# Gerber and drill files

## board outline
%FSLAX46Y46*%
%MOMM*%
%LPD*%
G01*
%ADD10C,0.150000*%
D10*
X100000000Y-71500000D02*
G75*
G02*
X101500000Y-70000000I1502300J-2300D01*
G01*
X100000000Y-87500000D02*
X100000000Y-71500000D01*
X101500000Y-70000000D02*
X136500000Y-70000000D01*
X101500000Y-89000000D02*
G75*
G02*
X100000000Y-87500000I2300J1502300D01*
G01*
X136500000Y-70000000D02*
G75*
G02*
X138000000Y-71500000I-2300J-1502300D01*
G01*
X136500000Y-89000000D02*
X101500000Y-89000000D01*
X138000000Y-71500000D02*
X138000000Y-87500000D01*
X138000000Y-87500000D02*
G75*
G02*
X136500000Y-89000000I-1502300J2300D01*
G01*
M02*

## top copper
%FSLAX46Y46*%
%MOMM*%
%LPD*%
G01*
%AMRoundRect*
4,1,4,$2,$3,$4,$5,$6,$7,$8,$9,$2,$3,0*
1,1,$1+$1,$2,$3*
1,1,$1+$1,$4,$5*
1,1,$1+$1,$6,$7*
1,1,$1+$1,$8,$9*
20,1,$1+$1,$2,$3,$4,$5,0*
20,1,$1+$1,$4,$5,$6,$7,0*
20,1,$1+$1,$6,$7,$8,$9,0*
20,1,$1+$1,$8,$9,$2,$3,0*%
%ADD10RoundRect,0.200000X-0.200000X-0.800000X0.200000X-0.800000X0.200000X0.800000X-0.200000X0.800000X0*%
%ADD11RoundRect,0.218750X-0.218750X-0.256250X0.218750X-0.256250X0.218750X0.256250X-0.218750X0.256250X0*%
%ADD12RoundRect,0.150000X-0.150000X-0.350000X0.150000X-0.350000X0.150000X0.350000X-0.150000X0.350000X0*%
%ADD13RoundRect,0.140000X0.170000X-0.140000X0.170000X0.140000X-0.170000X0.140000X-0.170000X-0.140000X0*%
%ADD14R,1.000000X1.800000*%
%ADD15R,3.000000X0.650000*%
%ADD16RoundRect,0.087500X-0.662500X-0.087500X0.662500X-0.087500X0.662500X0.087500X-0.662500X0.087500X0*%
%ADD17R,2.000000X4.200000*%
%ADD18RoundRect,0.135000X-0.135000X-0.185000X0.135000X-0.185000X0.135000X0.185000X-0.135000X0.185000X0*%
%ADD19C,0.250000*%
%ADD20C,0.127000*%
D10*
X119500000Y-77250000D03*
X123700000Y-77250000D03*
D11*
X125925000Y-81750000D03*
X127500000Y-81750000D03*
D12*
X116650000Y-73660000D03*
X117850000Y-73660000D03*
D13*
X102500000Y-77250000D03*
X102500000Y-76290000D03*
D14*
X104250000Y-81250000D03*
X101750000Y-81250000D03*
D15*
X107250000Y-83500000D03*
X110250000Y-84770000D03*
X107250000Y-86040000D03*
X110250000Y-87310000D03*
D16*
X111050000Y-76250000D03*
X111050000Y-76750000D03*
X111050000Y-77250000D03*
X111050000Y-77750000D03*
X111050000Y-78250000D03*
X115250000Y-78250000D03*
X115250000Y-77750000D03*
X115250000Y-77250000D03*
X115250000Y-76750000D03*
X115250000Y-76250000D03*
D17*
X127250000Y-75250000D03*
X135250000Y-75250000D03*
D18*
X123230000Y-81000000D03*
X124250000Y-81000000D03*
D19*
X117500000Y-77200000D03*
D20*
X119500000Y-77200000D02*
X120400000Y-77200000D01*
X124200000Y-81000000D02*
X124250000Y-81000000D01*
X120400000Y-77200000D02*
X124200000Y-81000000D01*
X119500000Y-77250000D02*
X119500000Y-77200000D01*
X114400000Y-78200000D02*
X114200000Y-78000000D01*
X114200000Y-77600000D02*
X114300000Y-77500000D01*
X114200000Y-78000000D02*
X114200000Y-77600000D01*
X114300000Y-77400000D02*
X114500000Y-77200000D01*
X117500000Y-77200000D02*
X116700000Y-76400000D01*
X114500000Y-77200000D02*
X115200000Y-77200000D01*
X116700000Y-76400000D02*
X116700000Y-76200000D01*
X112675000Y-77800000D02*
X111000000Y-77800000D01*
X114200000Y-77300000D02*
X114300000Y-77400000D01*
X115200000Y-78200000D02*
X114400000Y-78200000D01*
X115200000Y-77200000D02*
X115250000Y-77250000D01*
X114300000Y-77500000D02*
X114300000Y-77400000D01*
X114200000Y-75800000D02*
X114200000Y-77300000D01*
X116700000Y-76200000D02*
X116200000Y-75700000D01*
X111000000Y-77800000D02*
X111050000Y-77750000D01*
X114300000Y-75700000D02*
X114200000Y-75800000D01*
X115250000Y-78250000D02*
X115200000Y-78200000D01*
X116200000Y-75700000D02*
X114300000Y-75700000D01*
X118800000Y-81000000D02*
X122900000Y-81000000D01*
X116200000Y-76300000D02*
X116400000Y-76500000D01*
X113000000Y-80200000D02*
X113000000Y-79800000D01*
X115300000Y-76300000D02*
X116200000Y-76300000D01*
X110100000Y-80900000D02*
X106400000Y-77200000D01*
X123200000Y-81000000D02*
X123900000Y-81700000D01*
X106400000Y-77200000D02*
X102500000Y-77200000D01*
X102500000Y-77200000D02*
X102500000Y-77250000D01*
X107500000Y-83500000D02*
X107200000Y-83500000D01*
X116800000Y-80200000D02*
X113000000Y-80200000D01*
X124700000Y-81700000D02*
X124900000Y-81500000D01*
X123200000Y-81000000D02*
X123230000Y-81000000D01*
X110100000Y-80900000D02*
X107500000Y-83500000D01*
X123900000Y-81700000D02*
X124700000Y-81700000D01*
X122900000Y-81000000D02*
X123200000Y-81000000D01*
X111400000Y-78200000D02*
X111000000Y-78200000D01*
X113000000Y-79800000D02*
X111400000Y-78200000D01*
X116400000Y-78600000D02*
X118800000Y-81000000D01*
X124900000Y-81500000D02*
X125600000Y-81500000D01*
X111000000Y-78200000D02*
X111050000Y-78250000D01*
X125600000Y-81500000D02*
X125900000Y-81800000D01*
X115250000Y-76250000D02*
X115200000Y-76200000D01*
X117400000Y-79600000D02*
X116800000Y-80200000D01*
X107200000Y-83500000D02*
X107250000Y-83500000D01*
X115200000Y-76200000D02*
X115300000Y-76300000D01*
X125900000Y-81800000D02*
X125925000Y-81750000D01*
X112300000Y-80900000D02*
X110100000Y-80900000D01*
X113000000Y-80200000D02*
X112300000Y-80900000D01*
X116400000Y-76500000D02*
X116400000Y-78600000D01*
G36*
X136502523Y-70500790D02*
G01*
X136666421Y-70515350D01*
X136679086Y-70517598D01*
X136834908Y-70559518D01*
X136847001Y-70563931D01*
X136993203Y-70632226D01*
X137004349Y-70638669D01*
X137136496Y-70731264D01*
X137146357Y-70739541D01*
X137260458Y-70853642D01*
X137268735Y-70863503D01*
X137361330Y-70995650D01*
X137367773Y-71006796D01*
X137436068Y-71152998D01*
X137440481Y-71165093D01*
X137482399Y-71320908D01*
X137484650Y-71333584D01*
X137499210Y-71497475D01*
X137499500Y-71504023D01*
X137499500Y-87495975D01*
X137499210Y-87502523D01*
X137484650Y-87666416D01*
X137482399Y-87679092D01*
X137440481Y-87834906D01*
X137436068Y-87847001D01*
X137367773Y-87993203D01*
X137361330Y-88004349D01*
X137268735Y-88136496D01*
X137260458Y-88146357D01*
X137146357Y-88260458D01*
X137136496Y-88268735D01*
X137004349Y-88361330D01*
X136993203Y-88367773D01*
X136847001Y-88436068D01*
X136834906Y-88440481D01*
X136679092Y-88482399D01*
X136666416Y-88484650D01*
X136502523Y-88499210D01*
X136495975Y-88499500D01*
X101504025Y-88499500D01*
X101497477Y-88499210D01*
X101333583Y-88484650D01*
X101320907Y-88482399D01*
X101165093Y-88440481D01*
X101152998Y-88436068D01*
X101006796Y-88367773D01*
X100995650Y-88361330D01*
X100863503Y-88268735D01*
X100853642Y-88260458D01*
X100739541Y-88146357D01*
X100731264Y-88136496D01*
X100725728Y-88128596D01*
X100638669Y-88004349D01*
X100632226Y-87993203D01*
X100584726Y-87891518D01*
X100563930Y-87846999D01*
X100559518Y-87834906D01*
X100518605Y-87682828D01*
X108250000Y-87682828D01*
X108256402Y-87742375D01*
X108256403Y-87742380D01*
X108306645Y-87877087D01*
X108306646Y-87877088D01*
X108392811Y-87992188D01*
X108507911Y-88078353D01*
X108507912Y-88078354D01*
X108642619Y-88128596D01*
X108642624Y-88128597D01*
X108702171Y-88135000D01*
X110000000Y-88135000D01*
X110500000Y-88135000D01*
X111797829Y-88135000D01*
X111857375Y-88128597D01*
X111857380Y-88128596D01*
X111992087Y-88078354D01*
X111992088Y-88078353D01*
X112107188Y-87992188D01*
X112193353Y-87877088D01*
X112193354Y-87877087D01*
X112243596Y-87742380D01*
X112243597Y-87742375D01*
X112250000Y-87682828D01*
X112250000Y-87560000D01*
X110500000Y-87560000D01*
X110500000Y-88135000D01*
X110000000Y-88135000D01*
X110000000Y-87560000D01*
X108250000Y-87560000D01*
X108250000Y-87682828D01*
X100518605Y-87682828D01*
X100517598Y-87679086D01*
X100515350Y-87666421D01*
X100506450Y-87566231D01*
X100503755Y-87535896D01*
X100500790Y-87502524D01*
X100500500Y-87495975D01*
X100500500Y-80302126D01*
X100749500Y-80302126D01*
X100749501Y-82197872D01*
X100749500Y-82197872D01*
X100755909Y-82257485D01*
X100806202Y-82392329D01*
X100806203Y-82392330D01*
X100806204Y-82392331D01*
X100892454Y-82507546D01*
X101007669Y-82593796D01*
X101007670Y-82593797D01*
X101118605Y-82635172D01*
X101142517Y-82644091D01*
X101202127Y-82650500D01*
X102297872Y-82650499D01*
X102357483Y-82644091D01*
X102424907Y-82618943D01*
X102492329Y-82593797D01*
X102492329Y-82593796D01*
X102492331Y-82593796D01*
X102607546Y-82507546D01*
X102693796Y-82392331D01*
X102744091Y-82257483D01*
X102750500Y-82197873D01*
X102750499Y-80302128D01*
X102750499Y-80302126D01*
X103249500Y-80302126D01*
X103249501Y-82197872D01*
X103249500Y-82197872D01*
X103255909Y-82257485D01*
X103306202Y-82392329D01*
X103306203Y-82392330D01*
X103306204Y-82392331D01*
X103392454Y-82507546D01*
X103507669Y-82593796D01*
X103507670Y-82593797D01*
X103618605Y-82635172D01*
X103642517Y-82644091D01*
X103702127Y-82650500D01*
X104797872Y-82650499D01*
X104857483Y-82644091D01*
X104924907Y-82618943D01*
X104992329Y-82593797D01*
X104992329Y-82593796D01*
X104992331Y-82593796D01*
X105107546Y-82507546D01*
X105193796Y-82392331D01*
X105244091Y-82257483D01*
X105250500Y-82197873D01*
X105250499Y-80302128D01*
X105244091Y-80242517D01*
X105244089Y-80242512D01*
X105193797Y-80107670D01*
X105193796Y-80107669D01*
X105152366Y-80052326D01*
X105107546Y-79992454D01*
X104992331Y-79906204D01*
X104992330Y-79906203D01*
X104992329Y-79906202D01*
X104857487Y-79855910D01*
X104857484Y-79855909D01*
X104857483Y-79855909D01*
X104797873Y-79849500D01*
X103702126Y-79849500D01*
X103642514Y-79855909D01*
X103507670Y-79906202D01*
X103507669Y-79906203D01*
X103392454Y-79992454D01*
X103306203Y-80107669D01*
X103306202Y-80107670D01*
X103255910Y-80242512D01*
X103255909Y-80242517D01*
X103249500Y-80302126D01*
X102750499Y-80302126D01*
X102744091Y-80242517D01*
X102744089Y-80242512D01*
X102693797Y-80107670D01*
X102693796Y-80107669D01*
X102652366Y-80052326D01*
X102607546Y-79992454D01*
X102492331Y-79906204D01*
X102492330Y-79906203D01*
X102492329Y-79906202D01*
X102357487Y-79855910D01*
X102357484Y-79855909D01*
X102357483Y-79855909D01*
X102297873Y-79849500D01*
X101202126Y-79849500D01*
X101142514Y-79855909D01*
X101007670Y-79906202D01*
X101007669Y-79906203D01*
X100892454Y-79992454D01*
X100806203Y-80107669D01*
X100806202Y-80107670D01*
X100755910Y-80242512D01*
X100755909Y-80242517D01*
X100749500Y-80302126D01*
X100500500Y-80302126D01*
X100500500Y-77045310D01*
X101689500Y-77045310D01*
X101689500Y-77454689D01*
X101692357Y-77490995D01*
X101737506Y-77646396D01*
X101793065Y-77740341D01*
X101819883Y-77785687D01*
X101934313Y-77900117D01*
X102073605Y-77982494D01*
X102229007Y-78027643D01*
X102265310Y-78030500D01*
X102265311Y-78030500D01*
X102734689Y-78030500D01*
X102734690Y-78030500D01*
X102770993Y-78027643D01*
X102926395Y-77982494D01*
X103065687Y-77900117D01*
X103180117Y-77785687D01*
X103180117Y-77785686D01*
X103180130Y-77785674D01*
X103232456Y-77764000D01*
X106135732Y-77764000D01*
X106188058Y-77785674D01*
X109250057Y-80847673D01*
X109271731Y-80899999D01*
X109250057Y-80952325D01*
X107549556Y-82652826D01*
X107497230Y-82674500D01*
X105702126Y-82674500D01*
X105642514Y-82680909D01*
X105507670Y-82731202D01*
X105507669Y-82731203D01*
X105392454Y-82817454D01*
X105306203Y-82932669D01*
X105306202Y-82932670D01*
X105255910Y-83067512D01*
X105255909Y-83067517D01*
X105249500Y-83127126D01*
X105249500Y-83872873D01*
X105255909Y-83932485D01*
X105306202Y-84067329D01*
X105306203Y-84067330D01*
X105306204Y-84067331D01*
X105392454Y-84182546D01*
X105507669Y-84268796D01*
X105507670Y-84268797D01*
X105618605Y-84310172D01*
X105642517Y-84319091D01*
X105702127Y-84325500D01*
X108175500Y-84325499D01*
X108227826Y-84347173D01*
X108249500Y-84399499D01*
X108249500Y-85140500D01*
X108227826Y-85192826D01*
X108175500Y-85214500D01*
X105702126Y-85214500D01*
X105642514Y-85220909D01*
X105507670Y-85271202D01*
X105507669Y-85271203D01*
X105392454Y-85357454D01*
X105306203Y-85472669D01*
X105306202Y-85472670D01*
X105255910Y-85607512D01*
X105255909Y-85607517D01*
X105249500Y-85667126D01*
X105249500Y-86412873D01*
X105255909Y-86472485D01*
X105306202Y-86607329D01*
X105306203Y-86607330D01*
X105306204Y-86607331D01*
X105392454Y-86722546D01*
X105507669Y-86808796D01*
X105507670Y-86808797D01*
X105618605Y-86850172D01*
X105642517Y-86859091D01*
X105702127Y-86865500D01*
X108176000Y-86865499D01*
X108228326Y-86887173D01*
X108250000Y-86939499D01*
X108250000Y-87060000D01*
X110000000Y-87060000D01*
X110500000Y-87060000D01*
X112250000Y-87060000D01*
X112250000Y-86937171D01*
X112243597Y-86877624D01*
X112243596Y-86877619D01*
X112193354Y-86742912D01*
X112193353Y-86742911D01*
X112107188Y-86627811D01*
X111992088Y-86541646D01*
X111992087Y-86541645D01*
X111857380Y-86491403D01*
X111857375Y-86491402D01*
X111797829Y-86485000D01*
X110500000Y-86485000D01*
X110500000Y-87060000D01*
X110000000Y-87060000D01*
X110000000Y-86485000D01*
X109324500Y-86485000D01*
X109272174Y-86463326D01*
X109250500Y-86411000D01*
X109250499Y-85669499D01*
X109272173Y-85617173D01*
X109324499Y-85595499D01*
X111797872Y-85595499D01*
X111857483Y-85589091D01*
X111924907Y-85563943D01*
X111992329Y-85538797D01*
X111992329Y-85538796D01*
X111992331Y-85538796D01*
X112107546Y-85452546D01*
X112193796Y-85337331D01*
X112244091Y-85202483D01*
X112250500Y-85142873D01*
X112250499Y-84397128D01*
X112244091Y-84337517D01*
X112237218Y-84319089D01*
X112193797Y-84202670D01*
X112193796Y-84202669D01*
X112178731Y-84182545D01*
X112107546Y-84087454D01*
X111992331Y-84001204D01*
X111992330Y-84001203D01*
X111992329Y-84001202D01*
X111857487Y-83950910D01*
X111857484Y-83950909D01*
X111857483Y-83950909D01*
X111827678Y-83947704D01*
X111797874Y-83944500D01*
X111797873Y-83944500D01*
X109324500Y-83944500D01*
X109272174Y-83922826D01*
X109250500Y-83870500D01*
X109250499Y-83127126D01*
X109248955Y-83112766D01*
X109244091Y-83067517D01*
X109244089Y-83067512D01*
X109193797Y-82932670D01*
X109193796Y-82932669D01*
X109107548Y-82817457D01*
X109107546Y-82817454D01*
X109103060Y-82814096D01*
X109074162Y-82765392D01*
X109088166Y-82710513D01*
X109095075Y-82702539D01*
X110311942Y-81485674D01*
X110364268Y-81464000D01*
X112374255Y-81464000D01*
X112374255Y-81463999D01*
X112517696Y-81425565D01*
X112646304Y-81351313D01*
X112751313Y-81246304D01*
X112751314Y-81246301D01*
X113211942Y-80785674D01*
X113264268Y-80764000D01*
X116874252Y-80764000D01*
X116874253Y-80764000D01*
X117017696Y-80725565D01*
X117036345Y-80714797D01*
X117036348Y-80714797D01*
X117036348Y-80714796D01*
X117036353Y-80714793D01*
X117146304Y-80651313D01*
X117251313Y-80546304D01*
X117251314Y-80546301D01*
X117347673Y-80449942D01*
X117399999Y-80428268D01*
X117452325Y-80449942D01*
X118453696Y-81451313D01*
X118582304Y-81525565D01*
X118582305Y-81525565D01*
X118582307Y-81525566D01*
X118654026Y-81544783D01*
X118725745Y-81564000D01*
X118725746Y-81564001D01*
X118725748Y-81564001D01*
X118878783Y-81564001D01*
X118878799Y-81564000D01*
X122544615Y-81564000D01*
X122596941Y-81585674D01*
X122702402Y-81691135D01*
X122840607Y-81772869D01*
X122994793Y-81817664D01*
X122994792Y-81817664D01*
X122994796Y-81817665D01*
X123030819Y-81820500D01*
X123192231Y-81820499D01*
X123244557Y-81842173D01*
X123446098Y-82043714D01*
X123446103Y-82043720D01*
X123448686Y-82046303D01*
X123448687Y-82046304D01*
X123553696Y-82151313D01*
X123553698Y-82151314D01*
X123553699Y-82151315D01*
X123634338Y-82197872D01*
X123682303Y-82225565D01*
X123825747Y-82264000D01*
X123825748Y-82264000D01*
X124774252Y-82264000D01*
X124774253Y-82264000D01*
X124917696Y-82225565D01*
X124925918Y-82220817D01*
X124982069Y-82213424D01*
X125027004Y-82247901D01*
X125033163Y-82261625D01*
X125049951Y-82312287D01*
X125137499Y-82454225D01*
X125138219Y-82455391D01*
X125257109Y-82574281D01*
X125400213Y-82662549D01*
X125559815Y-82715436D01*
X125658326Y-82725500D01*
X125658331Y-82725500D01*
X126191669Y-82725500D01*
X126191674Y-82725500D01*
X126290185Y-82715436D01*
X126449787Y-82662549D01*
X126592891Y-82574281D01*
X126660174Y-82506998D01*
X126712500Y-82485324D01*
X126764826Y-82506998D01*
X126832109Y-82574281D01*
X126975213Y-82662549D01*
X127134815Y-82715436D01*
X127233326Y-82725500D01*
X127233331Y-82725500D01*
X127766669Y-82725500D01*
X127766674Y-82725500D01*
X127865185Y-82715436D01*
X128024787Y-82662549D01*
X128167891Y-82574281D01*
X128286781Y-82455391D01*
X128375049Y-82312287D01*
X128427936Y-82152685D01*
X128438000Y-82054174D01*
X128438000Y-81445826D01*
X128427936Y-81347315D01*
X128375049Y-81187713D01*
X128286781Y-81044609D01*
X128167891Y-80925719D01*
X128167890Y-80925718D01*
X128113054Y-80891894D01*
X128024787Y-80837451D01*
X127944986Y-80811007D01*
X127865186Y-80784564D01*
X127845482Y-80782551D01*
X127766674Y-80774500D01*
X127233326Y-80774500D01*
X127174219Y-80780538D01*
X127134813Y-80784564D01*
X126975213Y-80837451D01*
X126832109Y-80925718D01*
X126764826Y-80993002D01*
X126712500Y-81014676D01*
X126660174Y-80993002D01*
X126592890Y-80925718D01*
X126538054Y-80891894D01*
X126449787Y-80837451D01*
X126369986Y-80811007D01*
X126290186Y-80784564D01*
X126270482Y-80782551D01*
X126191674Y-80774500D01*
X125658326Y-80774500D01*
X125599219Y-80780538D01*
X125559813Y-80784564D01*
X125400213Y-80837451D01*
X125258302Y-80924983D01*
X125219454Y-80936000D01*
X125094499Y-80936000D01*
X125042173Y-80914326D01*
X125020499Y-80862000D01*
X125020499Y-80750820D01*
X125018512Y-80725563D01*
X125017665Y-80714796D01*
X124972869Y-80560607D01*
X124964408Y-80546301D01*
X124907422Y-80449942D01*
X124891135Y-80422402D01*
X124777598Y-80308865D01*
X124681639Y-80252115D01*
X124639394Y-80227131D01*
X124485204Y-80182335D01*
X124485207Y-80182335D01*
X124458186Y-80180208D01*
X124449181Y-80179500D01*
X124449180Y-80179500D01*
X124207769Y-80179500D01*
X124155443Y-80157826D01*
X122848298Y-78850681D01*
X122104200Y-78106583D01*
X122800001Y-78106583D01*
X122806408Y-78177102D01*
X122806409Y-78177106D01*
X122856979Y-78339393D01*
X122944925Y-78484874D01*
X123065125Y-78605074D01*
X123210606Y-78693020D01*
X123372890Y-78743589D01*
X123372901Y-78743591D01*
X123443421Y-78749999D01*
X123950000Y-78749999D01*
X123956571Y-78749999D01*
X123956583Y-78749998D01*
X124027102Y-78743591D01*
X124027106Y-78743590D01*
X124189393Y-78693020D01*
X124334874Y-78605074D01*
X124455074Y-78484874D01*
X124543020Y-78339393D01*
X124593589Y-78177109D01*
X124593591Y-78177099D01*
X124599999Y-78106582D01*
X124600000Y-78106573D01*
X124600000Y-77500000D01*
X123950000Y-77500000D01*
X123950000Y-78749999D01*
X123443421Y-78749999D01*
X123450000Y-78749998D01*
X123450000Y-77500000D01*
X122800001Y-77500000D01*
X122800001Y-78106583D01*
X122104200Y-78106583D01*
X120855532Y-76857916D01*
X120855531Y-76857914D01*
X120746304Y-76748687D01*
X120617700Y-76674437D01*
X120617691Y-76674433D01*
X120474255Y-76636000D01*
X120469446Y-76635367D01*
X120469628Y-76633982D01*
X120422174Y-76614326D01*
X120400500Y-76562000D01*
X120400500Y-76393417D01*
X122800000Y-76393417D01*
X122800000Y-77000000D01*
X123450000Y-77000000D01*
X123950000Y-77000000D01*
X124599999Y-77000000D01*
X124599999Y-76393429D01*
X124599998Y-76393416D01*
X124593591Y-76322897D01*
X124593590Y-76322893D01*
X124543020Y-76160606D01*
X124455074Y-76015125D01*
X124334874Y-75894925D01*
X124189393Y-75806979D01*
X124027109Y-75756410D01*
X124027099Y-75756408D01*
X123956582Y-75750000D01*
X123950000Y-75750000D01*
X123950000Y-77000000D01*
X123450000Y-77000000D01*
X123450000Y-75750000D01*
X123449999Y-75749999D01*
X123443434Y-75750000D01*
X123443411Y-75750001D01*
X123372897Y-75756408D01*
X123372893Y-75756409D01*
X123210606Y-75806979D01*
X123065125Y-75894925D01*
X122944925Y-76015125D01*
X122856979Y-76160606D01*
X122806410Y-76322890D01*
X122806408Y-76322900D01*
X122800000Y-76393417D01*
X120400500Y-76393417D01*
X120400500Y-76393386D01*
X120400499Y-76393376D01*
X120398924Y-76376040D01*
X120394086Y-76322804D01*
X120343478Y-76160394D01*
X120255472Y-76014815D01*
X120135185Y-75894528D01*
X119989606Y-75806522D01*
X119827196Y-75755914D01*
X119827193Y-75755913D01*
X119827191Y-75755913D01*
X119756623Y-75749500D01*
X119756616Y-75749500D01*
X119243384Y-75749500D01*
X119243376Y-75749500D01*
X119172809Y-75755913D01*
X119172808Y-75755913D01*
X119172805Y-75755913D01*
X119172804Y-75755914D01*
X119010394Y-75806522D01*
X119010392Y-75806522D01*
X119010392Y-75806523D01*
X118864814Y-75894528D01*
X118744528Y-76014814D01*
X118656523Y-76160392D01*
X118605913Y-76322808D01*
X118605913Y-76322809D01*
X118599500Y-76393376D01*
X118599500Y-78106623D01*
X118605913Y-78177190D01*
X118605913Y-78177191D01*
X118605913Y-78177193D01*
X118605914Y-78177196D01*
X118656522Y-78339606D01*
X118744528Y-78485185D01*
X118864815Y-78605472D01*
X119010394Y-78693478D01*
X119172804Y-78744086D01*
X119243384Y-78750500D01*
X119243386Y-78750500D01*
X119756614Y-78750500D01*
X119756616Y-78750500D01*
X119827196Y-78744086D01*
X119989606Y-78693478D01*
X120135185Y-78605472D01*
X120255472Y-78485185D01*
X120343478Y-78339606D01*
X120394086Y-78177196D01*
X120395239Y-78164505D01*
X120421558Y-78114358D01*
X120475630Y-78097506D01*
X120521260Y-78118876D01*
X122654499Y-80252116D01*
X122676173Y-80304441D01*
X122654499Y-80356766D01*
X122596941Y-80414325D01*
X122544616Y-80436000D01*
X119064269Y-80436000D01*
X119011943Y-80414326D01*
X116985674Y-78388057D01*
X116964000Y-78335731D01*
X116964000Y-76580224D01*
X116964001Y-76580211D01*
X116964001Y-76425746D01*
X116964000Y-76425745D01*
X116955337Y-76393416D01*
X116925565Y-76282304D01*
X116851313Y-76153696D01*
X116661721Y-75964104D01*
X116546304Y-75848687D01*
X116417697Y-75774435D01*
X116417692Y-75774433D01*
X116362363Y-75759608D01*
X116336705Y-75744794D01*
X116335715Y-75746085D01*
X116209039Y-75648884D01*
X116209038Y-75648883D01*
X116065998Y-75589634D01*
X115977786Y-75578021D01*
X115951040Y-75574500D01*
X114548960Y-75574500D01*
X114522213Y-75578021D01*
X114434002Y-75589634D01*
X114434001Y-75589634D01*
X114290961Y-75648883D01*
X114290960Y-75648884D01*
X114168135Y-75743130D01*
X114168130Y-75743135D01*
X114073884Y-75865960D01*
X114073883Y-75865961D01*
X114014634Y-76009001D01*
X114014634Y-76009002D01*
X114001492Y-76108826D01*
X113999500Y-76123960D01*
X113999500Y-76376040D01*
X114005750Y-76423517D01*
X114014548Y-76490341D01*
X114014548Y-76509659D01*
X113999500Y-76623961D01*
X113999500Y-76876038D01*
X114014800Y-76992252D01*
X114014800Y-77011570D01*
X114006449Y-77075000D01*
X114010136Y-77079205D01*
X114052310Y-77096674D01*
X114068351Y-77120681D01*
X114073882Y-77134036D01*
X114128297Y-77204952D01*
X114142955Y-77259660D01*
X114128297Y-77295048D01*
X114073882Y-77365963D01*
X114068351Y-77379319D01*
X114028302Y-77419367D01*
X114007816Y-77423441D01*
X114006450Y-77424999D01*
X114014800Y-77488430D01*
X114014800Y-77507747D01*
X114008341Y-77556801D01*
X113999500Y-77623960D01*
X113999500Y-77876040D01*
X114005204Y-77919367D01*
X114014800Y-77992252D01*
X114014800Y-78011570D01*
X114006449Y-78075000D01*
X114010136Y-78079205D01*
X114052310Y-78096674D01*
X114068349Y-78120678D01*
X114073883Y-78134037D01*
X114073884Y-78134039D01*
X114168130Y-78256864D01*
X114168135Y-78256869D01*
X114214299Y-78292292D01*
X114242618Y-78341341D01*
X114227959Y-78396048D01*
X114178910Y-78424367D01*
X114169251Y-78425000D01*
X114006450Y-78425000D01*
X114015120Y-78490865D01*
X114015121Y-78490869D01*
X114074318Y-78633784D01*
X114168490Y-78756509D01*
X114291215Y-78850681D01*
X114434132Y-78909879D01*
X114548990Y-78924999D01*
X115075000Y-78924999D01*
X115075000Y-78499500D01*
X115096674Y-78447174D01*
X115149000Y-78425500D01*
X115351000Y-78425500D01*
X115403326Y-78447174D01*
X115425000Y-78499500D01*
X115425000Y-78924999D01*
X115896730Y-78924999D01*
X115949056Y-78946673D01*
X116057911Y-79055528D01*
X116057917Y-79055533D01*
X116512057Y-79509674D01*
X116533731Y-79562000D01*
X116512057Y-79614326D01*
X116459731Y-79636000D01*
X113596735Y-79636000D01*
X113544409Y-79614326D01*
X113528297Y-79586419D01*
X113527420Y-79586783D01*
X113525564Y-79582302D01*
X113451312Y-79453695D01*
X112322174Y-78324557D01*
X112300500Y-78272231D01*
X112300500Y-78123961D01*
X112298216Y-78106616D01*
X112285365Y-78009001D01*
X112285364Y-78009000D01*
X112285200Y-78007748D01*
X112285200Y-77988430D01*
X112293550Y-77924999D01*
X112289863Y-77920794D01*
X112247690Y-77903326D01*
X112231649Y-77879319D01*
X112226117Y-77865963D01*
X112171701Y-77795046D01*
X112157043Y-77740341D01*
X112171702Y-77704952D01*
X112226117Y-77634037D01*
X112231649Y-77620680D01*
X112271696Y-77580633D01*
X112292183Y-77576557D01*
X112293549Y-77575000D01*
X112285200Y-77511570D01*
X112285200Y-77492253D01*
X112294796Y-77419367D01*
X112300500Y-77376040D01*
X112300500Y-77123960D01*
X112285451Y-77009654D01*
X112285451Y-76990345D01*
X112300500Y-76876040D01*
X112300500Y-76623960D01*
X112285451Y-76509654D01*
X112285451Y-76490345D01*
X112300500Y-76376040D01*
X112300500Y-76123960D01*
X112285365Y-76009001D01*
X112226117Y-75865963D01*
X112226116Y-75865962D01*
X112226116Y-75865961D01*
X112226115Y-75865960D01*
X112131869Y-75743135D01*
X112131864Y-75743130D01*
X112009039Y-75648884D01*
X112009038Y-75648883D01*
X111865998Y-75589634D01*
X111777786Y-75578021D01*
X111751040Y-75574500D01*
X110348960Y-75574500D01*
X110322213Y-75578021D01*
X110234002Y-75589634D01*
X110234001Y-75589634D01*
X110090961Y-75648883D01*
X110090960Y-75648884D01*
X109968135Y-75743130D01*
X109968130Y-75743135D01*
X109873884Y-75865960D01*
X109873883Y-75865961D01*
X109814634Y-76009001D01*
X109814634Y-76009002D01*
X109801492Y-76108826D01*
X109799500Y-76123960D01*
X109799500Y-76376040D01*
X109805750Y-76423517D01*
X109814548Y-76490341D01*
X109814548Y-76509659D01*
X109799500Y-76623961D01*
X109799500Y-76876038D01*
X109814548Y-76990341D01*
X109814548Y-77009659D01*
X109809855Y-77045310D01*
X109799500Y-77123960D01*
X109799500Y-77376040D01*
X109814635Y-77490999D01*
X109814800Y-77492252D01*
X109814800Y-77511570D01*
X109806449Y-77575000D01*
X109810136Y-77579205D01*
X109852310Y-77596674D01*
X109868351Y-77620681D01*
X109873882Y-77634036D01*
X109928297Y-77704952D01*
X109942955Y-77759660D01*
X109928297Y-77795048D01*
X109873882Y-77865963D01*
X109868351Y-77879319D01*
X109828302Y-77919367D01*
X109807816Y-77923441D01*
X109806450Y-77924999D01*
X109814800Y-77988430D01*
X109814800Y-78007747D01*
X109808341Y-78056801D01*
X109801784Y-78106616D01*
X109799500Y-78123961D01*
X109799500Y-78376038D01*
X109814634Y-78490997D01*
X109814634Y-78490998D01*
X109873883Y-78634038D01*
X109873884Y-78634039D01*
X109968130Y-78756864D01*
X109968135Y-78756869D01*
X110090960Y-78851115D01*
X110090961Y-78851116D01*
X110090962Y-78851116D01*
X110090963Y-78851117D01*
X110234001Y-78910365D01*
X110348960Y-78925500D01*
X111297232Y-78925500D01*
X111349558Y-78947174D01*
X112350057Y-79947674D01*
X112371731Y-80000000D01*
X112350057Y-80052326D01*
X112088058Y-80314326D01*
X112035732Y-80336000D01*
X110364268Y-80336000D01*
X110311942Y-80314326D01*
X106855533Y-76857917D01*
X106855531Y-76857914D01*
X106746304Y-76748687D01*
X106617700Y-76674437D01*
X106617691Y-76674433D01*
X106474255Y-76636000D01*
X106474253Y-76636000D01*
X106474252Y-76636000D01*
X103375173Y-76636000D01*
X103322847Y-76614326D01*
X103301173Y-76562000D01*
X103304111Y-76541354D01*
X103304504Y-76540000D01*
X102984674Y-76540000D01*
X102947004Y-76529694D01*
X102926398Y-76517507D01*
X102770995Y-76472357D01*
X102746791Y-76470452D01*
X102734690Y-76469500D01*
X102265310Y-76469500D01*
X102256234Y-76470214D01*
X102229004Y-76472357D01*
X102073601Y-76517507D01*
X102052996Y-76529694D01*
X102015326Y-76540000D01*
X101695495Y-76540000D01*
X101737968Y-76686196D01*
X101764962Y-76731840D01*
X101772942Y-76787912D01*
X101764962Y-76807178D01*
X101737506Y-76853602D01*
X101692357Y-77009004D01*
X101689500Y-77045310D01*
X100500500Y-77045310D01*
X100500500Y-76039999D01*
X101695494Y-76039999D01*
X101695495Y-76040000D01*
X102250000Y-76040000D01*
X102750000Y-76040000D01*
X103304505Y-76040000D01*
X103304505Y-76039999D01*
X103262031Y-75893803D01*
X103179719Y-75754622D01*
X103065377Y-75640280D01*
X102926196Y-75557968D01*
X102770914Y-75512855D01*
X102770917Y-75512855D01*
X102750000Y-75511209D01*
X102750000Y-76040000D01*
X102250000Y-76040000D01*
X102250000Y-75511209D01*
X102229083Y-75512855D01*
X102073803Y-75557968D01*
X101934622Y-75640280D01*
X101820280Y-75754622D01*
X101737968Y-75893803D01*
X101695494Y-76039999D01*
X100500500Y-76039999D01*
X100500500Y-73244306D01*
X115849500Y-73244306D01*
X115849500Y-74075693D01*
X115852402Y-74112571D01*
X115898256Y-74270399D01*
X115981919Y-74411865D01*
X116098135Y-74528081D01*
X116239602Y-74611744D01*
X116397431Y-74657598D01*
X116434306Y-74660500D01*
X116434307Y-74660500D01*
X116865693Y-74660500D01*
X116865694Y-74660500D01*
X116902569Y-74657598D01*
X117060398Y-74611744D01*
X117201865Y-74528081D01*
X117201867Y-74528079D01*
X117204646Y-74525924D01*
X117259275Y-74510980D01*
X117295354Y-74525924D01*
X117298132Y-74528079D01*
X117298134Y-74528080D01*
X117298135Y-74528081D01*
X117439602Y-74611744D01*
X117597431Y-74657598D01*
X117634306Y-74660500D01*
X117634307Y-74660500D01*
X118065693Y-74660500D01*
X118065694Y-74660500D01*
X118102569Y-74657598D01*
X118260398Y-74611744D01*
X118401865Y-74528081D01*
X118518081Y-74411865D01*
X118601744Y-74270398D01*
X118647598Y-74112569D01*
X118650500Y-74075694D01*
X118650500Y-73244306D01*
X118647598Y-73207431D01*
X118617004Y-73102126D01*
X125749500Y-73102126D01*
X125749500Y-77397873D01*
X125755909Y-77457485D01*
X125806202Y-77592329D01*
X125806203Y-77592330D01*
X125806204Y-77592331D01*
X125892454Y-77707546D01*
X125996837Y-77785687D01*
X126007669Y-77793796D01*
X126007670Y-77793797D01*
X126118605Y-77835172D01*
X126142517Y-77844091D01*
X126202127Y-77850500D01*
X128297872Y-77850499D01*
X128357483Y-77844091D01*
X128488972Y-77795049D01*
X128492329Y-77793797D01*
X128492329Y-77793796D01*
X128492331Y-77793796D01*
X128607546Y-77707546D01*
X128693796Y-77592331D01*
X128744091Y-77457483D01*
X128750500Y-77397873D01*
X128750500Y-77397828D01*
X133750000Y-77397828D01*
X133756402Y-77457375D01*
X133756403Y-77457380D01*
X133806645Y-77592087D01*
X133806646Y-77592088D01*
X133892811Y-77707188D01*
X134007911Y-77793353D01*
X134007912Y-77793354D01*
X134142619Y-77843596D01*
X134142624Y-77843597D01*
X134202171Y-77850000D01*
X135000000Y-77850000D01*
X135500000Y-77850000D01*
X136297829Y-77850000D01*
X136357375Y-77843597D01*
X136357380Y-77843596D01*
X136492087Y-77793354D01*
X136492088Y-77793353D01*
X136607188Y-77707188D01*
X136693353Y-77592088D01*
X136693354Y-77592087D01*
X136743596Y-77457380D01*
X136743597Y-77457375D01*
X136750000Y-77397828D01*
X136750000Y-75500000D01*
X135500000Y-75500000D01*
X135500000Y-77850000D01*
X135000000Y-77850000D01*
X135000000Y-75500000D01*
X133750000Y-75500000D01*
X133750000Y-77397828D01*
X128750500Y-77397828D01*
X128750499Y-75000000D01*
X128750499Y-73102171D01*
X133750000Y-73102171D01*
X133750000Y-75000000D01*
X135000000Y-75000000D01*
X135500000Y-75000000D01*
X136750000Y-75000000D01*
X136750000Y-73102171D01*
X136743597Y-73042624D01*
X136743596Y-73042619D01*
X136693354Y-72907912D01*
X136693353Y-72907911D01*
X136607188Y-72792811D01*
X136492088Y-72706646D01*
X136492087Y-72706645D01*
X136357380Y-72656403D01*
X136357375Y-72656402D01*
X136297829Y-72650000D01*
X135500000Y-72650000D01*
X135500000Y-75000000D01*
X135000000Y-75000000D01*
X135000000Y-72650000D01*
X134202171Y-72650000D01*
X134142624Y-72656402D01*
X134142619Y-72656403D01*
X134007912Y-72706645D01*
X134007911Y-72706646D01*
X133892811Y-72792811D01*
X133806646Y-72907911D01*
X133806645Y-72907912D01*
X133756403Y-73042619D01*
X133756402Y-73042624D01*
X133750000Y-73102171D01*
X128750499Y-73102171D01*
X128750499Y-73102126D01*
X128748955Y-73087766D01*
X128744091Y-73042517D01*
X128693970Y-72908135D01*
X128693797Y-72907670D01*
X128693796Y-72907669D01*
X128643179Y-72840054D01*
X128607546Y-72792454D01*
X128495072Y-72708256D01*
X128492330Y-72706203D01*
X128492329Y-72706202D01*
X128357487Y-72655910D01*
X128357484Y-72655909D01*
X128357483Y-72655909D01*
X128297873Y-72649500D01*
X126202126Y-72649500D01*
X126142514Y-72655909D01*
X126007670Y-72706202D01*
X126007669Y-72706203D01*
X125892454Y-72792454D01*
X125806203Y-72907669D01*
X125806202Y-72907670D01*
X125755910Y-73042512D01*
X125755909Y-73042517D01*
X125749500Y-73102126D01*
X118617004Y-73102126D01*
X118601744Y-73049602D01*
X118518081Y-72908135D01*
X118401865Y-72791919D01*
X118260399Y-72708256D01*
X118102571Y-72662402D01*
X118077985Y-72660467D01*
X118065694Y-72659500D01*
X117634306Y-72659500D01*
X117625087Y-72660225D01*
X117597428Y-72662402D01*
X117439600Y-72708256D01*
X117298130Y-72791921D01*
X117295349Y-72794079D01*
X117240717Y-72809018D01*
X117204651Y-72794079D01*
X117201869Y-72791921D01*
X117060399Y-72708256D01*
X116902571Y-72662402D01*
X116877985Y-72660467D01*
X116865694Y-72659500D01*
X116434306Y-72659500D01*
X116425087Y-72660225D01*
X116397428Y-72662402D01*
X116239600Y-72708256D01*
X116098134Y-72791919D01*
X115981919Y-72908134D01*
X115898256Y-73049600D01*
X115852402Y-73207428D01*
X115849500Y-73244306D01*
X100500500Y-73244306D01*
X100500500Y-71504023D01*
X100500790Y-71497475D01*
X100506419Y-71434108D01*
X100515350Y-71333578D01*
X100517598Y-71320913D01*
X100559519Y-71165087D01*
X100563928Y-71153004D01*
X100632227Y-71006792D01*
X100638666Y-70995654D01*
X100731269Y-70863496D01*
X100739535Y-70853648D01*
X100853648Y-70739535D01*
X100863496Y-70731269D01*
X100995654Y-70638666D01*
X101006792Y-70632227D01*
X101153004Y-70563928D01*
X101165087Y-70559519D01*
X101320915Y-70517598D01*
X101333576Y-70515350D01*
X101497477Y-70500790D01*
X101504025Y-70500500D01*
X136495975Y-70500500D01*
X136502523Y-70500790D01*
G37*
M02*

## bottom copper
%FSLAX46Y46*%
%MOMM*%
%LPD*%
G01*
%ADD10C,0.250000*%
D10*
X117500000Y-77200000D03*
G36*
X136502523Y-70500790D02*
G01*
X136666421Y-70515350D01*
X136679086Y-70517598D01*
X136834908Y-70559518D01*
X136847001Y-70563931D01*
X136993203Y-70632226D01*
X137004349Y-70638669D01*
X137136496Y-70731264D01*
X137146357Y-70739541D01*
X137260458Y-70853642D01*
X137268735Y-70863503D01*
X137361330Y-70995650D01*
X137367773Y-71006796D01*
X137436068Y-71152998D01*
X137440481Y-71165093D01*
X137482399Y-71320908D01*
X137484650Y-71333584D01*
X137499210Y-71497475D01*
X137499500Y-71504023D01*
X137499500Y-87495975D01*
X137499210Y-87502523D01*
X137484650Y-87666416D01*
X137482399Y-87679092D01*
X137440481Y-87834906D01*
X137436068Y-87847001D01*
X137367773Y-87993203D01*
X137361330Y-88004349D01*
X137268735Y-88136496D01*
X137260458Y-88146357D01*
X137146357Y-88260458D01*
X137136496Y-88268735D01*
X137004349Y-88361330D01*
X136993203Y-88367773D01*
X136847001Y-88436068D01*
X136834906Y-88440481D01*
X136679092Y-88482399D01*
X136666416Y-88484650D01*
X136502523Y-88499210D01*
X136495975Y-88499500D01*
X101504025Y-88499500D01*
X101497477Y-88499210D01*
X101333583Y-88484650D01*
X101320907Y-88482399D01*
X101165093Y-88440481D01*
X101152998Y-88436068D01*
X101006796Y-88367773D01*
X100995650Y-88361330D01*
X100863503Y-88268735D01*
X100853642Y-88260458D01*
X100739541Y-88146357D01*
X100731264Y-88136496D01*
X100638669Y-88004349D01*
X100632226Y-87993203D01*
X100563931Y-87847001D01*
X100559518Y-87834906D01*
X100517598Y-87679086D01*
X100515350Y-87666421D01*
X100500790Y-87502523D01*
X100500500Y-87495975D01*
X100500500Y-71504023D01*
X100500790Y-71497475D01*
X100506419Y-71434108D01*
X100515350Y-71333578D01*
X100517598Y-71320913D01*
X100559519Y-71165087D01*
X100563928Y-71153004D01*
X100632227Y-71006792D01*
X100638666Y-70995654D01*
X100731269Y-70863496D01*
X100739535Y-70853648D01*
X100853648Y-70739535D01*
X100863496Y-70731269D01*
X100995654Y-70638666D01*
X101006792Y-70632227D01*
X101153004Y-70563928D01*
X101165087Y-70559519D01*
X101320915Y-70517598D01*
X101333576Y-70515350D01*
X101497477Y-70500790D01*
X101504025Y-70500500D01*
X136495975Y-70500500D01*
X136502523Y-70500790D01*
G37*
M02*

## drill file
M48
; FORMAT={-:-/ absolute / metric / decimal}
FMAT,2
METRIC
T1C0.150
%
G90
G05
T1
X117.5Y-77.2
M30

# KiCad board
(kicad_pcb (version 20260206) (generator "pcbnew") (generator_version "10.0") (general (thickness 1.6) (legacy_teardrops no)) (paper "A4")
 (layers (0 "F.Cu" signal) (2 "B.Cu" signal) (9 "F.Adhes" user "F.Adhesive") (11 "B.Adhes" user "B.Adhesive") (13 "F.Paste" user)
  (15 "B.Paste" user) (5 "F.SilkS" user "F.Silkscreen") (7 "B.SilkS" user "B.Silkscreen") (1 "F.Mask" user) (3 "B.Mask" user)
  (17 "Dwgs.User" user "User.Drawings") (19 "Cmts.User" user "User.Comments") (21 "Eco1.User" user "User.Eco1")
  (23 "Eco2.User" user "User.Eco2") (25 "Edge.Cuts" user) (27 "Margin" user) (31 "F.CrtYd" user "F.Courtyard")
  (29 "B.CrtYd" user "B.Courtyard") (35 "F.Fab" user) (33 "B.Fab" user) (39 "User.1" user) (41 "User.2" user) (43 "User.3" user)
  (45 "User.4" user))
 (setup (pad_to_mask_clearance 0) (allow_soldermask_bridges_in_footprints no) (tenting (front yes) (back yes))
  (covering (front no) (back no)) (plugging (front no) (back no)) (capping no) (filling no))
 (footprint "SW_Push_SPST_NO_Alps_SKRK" (layer "F.Cu") (at 121.6 77.25)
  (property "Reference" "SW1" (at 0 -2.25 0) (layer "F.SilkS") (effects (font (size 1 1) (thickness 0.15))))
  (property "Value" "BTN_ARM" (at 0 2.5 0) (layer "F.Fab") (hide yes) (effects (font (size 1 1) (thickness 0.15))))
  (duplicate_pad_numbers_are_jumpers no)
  (pad "1" smd roundrect (at -2.1 0) (size 0.8 2) (layers "F.Cu" "F.Mask" "F.Paste") (roundrect_rratio 0.25) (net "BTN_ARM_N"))
  (pad "2" smd roundrect (at 2.1 0) (size 0.8 2) (layers "F.Cu" "F.Mask" "F.Paste") (roundrect_rratio 0.25) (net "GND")))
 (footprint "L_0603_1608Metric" (layer "F.Cu") (at 126.7125 81.75)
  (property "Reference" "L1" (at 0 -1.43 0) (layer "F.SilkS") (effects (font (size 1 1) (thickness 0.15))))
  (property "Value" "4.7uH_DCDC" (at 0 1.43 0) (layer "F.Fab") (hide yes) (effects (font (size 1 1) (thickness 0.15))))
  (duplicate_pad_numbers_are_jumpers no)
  (pad "1" smd roundrect (at -0.7875 0) (size 0.875 0.95) (layers "F.Cu" "F.Mask" "F.Paste") (roundrect_rratio 0.25) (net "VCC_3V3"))
  (pad "2" smd roundrect (at 0.7875 0) (size 0.875 0.95) (layers "F.Cu" "F.Mask" "F.Paste") (roundrect_rratio 0.25) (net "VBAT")))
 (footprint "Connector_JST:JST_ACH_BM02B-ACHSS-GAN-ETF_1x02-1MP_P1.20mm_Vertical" (layer "F.Cu") (at 117.25 73.66)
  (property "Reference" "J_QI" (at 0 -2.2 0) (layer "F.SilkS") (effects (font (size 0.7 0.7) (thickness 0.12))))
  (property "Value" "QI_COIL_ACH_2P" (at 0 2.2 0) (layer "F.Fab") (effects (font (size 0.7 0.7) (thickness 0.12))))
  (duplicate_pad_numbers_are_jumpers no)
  (pad "1" smd roundrect (at -0.6 0) (size 0.6 1) (layers "F.Cu" "F.Mask" "F.Paste") (roundrect_rratio 0.25) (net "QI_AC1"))
  (pad "2" smd roundrect (at 0.6 0) (size 0.6 1) (layers "F.Cu" "F.Mask" "F.Paste") (roundrect_rratio 0.25) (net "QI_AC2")))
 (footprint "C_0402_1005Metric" (layer "F.Cu") (at 102.5 76.77 90)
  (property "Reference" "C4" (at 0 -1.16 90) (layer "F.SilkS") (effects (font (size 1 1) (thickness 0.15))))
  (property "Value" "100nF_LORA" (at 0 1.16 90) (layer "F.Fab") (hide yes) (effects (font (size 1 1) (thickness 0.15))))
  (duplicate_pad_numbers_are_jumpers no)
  (pad "1" smd roundrect (at -0.48 0 90) (size 0.56 0.62) (layers "F.Cu" "F.Mask" "F.Paste") (roundrect_rratio 0.25) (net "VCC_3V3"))
  (pad "2" smd roundrect (at 0.48 0 90) (size 0.56 0.62) (layers "F.Cu" "F.Mask" "F.Paste") (roundrect_rratio 0.25) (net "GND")))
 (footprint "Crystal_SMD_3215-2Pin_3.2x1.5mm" (layer "F.Cu") (at 103 81.25)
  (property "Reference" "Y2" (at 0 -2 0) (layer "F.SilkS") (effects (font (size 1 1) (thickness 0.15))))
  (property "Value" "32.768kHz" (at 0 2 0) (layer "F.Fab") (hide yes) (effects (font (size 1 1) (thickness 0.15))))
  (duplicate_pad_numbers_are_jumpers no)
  (pad "1" smd rect (at 1.25 0) (size 1 1.8) (layers "F.Cu" "F.Mask" "F.Paste") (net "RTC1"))
  (pad "2" smd rect (at -1.25 0) (size 1 1.8) (layers "F.Cu" "F.Mask" "F.Paste") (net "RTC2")))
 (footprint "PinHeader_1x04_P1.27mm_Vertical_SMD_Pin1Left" (layer "F.Cu") (at 108.75 85.405)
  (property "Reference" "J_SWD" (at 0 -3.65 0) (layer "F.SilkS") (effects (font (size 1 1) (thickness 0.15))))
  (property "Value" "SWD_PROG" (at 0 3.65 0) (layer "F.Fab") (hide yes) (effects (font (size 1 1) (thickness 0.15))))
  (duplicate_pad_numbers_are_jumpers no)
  (pad "1" smd rect (at -1.5 -1.905) (size 3 0.65) (layers "F.Cu" "F.Mask" "F.Paste") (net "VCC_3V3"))
  (pad "2" smd rect (at 1.5 -0.635) (size 3 0.65) (layers "F.Cu" "F.Mask" "F.Paste") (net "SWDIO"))
  (pad "3" smd rect (at -1.5 0.635) (size 3 0.65) (layers "F.Cu" "F.Mask" "F.Paste") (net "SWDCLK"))
  (pad "4" smd rect (at 1.5 1.905) (size 3 0.65) (layers "F.Cu" "F.Mask" "F.Paste") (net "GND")))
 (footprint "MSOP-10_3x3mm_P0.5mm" (layer "F.Cu") (at 113.15 77.25)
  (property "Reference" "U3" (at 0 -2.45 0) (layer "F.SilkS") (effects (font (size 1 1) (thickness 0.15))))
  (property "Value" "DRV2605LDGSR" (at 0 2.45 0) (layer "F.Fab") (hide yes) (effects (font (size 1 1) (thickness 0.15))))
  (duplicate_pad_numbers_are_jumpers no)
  (pad "1" smd roundrect (at -2.1 -1) (size 1.5 0.35) (layers "F.Cu" "F.Mask" "F.Paste") (roundrect_rratio 0.25) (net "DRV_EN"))
  (pad "2" smd roundrect (at -2.1 -0.5) (size 1.5 0.35) (layers "F.Cu" "F.Mask" "F.Paste") (roundrect_rratio 0.25) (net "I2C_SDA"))
  (pad "3" smd roundrect (at -2.1 0) (size 1.5 0.35) (layers "F.Cu" "F.Mask" "F.Paste") (roundrect_rratio 0.25) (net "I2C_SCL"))
  (pad "4" smd roundrect (at -2.1 0.5) (size 1.5 0.35) (layers "F.Cu" "F.Mask" "F.Paste") (roundrect_rratio 0.25) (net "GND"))
  (pad "5" smd roundrect (at -2.1 1) (size 1.5 0.35) (layers "F.Cu" "F.Mask" "F.Paste") (roundrect_rratio 0.25) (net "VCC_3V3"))
  (pad "6" smd roundrect (at 2.1 1) (size 1.5 0.35) (layers "F.Cu" "F.Mask" "F.Paste") (roundrect_rratio 0.25) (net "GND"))
  (pad "7" smd roundrect (at 2.1 0.5) (size 1.5 0.35) (layers "F.Cu" "F.Mask" "F.Paste") (roundrect_rratio 0.25) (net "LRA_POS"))
  (pad "8" smd roundrect (at 2.1 0) (size 1.5 0.35) (layers "F.Cu" "F.Mask" "F.Paste") (roundrect_rratio 0.25) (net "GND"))
  (pad "9" smd roundrect (at 2.1 -0.5) (size 1.5 0.35) (layers "F.Cu" "F.Mask" "F.Paste") (roundrect_rratio 0.25) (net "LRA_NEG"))
  (pad "10" smd roundrect (at 2.1 -1) (size 1.5 0.35) (layers "F.Cu" "F.Mask" "F.Paste") (roundrect_rratio 0.25) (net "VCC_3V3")))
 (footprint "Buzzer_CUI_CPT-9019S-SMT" (layer "F.Cu") (at 131.25 75.25)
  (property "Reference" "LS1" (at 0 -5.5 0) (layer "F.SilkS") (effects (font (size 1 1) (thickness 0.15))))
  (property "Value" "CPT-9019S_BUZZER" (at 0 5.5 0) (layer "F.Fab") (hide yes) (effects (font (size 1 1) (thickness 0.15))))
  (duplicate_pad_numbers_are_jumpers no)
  (pad "1" smd rect (at -4 0) (size 2 4.2) (layers "F.Cu" "F.Mask" "F.Paste") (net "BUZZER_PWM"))
  (pad "2" smd rect (at 4 0) (size 2 4.2) (layers "F.Cu" "F.Mask" "F.Paste") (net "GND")))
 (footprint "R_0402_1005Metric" (layer "F.Cu") (at 123.74 81)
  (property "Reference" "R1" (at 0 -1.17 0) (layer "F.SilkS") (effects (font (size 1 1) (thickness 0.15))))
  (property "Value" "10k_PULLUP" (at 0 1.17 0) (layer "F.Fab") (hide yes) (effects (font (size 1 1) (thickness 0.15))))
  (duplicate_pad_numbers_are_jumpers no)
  (pad "1" smd roundrect (at -0.51 0) (size 0.54 0.64) (layers "F.Cu" "F.Mask" "F.Paste") (roundrect_rratio 0.25) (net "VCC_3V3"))
  (pad "2" smd roundrect (at 0.51 0) (size 0.54 0.64) (layers "F.Cu" "F.Mask" "F.Paste") (roundrect_rratio 0.25) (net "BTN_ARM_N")))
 (gr_arc (start 100 71.5) (mid 100.44 70.44) (end 101.5 70) (stroke (width 0.15) (type default)) (layer "Edge.Cuts"))
 (gr_line (start 100 87.5) (end 100 71.5) (stroke (width 0.15) (type default)) (layer "Edge.Cuts"))
 (gr_line (start 101.5 70) (end 136.5 70) (stroke (width 0.15) (type default)) (layer "Edge.Cuts"))
 (gr_arc (start 101.5 89) (mid 100.44 88.56) (end 100 87.5) (stroke (width 0.15) (type default)) (layer "Edge.Cuts"))
 (gr_arc (start 136.5 70) (mid 137.56 70.44) (end 138 71.5) (stroke (width 0.15) (type default)) (layer "Edge.Cuts"))
 (gr_line (start 136.5 89) (end 101.5 89) (stroke (width 0.15) (type default)) (layer "Edge.Cuts"))
 (gr_line (start 138 71.5) (end 138 87.5) (stroke (width 0.15) (type default)) (layer "Edge.Cuts"))
 (gr_arc (start 138 87.5) (mid 137.56 88.56) (end 136.5 89) (stroke (width 0.15) (type default)) (layer "Edge.Cuts"))
 (segment (start 119.5 77.2) (end 120.4 77.2) (width 0.127) (layer "F.Cu") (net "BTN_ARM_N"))
 (segment (start 124.2 81) (end 124.25 81) (width 0.127) (layer "F.Cu") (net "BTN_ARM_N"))
 (segment (start 120.4 77.2) (end 124.2 81) (width 0.127) (layer "F.Cu") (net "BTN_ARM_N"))
 (segment (start 119.5 77.25) (end 119.5 77.2) (width 0.127) (layer "F.Cu") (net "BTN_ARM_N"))
 (segment (start 114.4 78.2) (end 114.2 78) (width 0.127) (layer "F.Cu") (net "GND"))
 (segment (start 114.2 77.6) (end 114.3 77.5) (width 0.127) (layer "F.Cu") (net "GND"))
 (segment (start 114.2 78) (end 114.2 77.6) (width 0.127) (layer "F.Cu") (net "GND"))
 (segment (start 114.3 77.4) (end 114.5 77.2) (width 0.127) (layer "F.Cu") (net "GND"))
 (segment (start 117.5 77.2) (end 116.7 76.4) (width 0.127) (layer "F.Cu") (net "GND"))
 (segment (start 114.5 77.2) (end 115.2 77.2) (width 0.127) (layer "F.Cu") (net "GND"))
 (segment (start 116.7 76.4) (end 116.7 76.2) (width 0.127) (layer "F.Cu") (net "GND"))
 (segment (start 112.675 77.8) (end 111 77.8) (width 0.127) (layer "F.Cu") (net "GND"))
 (segment (start 114.2 77.3) (end 114.3 77.4) (width 0.127) (layer "F.Cu") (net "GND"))
 (segment (start 115.2 78.2) (end 114.4 78.2) (width 0.127) (layer "F.Cu") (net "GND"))
 (segment (start 115.2 77.2) (end 115.25 77.25) (width 0.127) (layer "F.Cu") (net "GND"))
 (segment (start 114.3 77.5) (end 114.3 77.4) (width 0.127) (layer "F.Cu") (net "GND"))
 (segment (start 114.2 75.8) (end 114.2 77.3) (width 0.127) (layer "F.Cu") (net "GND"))
 (segment (start 116.7 76.2) (end 116.2 75.7) (width 0.127) (layer "F.Cu") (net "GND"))
 (segment (start 111 77.8) (end 111.05 77.75) (width 0.127) (layer "F.Cu") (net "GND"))
 (segment (start 114.3 75.7) (end 114.2 75.8) (width 0.127) (layer "F.Cu") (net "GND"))
 (segment (start 115.25 78.25) (end 115.2 78.2) (width 0.127) (layer "F.Cu") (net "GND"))
 (segment (start 116.2 75.7) (end 114.3 75.7) (width 0.127) (layer "F.Cu") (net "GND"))
 (via (at 117.5 77.2) (size 0.25) (drill 0.15) (layers "F.Cu" "B.Cu") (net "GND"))
 (segment (start 118.8 81) (end 122.9 81) (width 0.127) (layer "F.Cu") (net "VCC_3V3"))
 (segment (start 116.2 76.3) (end 116.4 76.5) (width 0.127) (layer "F.Cu") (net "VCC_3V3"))
 (segment (start 113 80.2) (end 113 79.8) (width 0.127) (layer "F.Cu") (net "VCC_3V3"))
 (segment (start 115.3 76.3) (end 116.2 76.3) (width 0.127) (layer "F.Cu") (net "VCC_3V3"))
 (segment (start 110.1 80.9) (end 106.4 77.2) (width 0.127) (layer "F.Cu") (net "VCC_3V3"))
 (segment (start 123.2 81) (end 123.9 81.7) (width 0.127) (layer "F.Cu") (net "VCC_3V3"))
 (segment (start 106.4 77.2) (end 102.5 77.2) (width 0.127) (layer "F.Cu") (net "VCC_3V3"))
 (segment (start 102.5 77.2) (end 102.5 77.25) (width 0.127) (layer "F.Cu") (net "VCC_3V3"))
 (segment (start 107.5 83.5) (end 107.2 83.5) (width 0.127) (layer "F.Cu") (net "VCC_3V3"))
 (segment (start 116.8 80.2) (end 113 80.2) (width 0.127) (layer "F.Cu") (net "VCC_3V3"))
 (segment (start 124.7 81.7) (end 124.9 81.5) (width 0.127) (layer "F.Cu") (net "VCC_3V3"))
 (segment (start 123.2 81) (end 123.23 81) (width 0.127) (layer "F.Cu") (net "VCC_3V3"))
 (segment (start 110.1 80.9) (end 107.5 83.5) (width 0.127) (layer "F.Cu") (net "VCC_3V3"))
 (segment (start 123.9 81.7) (end 124.7 81.7) (width 0.127) (layer "F.Cu") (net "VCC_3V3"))
 (segment (start 122.9 81) (end 123.2 81) (width 0.127) (layer "F.Cu") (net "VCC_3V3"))
 (segment (start 111.4 78.2) (end 111 78.2) (width 0.127) (layer "F.Cu") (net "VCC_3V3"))
 (segment (start 113 79.8) (end 111.4 78.2) (width 0.127) (layer "F.Cu") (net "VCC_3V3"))
 (segment (start 116.4 78.6) (end 118.8 81) (width 0.127) (layer "F.Cu") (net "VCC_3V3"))
 (segment (start 124.9 81.5) (end 125.6 81.5) (width 0.127) (layer "F.Cu") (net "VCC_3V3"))
 (segment (start 111 78.2) (end 111.05 78.25) (width 0.127) (layer "F.Cu") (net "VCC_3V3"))
 (segment (start 125.6 81.5) (end 125.9 81.8) (width 0.127) (layer "F.Cu") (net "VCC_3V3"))
 (segment (start 115.25 76.25) (end 115.2 76.2) (width 0.127) (layer "F.Cu") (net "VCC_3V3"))
 (segment (start 117.4 79.6) (end 116.8 80.2) (width 0.127) (layer "F.Cu") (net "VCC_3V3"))
 (segment (start 107.2 83.5) (end 107.25 83.5) (width 0.127) (layer "F.Cu") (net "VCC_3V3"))
 (segment (start 115.2 76.2) (end 115.3 76.3) (width 0.127) (layer "F.Cu") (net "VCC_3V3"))
 (segment (start 125.9 81.8) (end 125.925 81.75) (width 0.127) (layer "F.Cu") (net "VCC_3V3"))
 (segment (start 112.3 80.9) (end 110.1 80.9) (width 0.127) (layer "F.Cu") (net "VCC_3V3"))
 (segment (start 113 80.2) (end 112.3 80.9) (width 0.127) (layer "F.Cu") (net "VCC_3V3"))
 (segment (start 116.4 76.5) (end 116.4 78.6) (width 0.127) (layer "F.Cu") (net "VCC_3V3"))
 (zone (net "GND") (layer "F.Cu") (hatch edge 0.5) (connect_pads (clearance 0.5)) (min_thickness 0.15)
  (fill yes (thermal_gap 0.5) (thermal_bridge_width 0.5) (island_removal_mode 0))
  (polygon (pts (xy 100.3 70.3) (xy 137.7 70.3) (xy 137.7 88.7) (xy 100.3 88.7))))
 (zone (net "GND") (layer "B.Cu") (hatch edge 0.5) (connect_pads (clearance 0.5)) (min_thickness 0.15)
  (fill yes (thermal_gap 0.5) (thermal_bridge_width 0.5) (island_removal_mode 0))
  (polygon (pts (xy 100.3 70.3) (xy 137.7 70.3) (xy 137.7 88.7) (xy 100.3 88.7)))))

